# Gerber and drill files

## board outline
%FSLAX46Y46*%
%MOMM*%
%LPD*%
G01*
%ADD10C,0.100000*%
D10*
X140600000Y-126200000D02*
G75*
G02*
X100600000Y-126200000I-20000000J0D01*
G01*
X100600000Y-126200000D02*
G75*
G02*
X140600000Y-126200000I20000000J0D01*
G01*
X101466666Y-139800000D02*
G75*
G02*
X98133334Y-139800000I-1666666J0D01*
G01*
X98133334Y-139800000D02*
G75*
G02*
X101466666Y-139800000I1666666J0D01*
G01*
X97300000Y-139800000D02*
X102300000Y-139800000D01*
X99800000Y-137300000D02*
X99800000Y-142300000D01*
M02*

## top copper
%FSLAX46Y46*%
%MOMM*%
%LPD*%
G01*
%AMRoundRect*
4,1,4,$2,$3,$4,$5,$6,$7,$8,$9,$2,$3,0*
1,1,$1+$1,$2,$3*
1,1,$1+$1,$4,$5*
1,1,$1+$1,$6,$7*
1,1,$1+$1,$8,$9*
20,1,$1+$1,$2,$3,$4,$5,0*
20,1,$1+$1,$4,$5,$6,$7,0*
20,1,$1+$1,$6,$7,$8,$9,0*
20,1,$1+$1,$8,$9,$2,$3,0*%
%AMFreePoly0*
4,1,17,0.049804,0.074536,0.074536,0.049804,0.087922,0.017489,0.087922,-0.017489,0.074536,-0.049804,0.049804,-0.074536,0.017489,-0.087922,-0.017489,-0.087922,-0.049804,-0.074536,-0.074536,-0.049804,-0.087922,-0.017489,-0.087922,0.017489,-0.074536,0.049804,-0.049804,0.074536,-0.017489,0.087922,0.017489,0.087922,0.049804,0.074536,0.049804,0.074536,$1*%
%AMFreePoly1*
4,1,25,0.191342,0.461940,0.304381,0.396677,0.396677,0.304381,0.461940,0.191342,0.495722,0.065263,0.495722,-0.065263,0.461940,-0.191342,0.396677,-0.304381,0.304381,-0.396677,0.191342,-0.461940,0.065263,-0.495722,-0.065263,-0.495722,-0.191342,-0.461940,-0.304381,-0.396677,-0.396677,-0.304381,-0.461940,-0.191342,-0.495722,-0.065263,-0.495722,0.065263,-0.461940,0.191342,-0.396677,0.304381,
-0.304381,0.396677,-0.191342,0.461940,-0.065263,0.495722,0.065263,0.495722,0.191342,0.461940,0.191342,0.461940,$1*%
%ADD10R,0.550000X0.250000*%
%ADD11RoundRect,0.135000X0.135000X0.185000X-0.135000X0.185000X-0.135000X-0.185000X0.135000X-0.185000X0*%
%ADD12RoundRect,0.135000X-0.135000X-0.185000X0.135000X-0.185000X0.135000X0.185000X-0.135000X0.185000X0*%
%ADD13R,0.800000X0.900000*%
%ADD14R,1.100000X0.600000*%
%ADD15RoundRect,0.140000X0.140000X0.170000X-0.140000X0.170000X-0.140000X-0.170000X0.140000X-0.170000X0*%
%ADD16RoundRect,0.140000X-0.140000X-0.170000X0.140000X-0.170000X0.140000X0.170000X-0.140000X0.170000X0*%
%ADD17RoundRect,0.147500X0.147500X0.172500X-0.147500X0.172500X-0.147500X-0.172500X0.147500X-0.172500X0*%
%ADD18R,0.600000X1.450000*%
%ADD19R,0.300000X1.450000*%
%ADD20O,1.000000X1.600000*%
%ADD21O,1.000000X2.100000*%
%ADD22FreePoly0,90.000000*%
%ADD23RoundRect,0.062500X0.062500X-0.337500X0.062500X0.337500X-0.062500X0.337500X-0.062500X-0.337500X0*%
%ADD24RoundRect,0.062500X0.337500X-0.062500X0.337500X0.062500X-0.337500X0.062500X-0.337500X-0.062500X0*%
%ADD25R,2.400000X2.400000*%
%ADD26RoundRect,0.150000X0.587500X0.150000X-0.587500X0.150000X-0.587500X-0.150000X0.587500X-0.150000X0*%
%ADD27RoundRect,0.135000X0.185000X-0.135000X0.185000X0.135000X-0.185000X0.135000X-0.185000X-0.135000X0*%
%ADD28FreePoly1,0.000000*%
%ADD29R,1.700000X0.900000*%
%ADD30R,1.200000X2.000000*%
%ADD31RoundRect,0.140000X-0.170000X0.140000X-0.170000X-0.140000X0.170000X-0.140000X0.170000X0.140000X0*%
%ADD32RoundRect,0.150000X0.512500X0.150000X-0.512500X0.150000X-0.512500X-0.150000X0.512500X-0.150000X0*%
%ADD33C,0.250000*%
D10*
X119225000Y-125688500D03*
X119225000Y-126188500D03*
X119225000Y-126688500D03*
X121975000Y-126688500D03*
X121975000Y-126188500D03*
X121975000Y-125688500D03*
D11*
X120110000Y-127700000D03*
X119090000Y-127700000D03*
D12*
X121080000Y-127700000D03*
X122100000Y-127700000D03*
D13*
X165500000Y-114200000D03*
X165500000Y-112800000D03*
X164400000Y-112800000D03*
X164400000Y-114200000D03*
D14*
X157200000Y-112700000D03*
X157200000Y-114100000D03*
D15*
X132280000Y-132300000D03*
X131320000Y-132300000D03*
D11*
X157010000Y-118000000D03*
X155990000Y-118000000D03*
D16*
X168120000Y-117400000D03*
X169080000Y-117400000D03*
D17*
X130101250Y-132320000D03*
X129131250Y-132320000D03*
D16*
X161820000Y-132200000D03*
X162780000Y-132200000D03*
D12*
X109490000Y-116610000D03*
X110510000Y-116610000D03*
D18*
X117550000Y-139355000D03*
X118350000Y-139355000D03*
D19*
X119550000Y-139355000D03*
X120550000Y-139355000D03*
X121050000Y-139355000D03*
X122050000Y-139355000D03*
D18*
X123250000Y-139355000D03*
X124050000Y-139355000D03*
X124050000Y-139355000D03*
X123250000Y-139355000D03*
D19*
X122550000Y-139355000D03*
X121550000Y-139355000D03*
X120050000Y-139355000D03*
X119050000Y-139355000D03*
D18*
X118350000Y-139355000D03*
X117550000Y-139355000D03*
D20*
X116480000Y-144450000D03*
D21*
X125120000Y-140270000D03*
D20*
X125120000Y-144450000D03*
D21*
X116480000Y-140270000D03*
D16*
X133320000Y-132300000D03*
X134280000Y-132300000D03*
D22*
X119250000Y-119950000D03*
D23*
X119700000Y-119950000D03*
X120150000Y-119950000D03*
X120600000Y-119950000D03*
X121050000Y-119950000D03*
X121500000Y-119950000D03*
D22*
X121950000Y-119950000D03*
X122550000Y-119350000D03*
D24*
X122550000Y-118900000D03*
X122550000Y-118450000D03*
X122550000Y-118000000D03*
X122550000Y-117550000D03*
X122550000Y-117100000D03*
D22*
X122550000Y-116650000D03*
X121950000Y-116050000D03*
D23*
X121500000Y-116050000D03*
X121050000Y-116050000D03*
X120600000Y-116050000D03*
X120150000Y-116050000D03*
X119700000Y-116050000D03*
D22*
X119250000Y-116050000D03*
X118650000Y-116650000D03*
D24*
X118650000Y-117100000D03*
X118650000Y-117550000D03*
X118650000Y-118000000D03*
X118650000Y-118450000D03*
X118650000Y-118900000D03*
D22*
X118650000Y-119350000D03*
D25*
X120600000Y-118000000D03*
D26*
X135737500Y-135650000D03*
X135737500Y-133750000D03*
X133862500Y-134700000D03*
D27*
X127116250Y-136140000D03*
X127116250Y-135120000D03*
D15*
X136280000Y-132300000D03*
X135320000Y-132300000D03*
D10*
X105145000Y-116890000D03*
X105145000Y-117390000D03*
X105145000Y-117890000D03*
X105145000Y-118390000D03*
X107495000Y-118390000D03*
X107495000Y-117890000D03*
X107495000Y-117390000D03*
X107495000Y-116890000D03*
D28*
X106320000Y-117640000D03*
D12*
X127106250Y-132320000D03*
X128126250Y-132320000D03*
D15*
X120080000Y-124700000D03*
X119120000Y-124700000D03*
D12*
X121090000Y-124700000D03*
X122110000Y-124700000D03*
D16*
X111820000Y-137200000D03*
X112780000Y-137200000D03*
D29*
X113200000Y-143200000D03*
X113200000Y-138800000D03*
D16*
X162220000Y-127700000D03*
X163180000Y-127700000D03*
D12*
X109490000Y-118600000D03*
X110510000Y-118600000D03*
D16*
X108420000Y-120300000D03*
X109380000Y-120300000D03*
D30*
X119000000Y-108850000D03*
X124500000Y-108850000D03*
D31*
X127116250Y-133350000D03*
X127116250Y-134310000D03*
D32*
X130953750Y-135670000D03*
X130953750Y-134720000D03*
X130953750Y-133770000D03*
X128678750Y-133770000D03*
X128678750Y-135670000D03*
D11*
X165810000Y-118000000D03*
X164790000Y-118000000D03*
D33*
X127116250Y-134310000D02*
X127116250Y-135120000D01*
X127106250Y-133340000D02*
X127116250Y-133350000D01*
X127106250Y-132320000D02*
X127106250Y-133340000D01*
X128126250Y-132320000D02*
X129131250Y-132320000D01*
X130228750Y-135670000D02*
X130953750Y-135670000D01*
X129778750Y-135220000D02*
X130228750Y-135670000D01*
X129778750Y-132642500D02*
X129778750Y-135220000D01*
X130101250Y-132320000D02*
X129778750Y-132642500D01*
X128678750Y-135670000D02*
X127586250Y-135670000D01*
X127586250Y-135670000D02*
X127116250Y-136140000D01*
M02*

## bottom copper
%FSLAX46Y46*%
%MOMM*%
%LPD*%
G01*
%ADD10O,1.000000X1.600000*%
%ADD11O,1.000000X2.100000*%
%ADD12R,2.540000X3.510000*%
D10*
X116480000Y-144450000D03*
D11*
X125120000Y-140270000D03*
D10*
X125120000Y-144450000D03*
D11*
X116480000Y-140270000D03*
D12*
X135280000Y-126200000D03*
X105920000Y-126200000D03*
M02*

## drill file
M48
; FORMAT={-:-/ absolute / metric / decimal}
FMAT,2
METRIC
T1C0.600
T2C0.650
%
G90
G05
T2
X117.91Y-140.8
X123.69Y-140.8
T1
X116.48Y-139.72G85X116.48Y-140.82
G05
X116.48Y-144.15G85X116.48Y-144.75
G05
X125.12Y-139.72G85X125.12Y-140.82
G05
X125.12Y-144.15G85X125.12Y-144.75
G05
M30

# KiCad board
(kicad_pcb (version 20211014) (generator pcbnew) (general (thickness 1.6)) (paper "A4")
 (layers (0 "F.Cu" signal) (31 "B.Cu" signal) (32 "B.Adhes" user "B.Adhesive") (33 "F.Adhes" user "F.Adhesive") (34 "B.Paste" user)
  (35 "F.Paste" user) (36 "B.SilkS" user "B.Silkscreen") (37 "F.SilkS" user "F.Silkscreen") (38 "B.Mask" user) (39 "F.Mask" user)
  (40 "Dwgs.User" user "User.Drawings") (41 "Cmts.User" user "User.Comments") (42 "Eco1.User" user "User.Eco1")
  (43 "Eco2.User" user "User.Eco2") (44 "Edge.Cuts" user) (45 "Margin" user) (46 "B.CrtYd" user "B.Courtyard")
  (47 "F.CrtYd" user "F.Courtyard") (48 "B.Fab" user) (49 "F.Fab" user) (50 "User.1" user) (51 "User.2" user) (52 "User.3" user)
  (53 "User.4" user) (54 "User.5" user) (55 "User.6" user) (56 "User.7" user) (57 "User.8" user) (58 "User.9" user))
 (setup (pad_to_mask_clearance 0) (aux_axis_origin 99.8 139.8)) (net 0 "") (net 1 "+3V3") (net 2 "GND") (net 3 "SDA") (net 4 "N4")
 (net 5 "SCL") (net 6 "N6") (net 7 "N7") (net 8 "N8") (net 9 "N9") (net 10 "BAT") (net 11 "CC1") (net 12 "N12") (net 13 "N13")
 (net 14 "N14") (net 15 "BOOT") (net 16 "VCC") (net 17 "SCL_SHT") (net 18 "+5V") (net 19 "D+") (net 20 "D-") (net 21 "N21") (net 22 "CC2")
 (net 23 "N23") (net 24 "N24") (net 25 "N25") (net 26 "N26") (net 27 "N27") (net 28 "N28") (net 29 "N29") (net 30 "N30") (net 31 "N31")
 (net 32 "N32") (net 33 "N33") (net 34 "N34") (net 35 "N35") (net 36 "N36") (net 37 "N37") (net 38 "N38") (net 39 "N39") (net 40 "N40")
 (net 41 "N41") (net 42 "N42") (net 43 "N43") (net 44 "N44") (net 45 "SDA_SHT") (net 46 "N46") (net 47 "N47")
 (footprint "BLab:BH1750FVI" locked (layer "F.Cu") (at 120.6 126.1885)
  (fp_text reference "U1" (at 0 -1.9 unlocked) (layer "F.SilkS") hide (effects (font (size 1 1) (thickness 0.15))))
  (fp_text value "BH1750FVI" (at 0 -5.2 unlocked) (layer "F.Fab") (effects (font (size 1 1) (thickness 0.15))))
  (pad "1" smd rect locked (at -1.375 -0.5) (size 0.55 0.25) (layers "F.Cu" "F.Paste" "F.Mask") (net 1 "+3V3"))
  (pad "2" smd rect locked (at -1.375 0) (size 0.55 0.25) (layers "F.Cu" "F.Paste" "F.Mask") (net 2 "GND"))
  (pad "3" smd rect locked (at -1.375 0.5) (size 0.55 0.25) (layers "F.Cu" "F.Paste" "F.Mask") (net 2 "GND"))
  (pad "4" smd rect locked (at 1.375 0.5) (size 0.55 0.25) (layers "F.Cu" "F.Paste" "F.Mask") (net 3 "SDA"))
  (pad "5" smd rect locked (at 1.375 0) (size 0.55 0.25) (layers "F.Cu" "F.Paste" "F.Mask") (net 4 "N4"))
  (pad "6" smd rect locked (at 1.375 -0.5) (size 0.55 0.25) (layers "F.Cu" "F.Paste" "F.Mask") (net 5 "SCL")))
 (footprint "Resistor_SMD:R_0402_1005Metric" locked (layer "F.Cu") (at 119.6 127.7 180)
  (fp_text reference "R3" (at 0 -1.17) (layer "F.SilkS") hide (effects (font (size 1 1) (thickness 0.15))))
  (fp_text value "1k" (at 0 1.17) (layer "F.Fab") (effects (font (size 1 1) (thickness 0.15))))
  (pad "1" smd roundrect locked (at -0.51 0 180) (size 0.54 0.64) (layers "F.Cu" "F.Paste" "F.Mask") (roundrect_rratio 0.25) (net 1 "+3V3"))
  (pad "2" smd roundrect locked (at 0.51 0 180) (size 0.54 0.64) (layers "F.Cu" "F.Paste" "F.Mask") (roundrect_rratio 0.25) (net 4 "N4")))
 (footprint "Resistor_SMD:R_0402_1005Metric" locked (layer "F.Cu") (at 121.59 127.7)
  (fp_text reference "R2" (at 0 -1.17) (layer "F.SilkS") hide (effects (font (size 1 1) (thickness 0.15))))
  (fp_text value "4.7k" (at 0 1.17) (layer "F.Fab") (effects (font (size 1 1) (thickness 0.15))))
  (pad "1" smd roundrect locked (at -0.51 0) (size 0.54 0.64) (layers "F.Cu" "F.Paste" "F.Mask") (roundrect_rratio 0.25) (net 1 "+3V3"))
  (pad "2" smd roundrect locked (at 0.51 0) (size 0.54 0.64) (layers "F.Cu" "F.Paste" "F.Mask") (roundrect_rratio 0.25) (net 3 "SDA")))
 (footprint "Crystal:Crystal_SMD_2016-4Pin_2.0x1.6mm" (layer "F.Cu") (at 164.95 113.5 90)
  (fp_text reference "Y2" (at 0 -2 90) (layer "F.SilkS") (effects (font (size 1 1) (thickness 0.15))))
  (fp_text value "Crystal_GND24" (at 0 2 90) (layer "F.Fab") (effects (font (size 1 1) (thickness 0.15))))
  (pad "1" smd rect (at -0.7 0.55 90) (size 0.9 0.8) (layers "F.Cu" "F.Paste" "F.Mask") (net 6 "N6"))
  (pad "2" smd rect (at 0.7 0.55 90) (size 0.9 0.8) (layers "F.Cu" "F.Paste" "F.Mask") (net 2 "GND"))
  (pad "3" smd rect (at 0.7 -0.55 90) (size 0.9 0.8) (layers "F.Cu" "F.Paste" "F.Mask") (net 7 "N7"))
  (pad "4" smd rect (at -0.7 -0.55 90) (size 0.9 0.8) (layers "F.Cu" "F.Paste" "F.Mask") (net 2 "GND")))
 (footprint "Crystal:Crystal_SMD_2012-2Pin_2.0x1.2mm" (layer "F.Cu") (at 157.2 113.4 -90)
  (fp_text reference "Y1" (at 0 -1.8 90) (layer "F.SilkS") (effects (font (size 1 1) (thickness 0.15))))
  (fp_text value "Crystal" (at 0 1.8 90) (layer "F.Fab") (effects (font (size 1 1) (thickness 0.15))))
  (pad "1" smd rect (at -0.7 0 270) (size 0.6 1.1) (layers "F.Cu" "F.Paste" "F.Mask") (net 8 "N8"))
  (pad "2" smd rect (at 0.7 0 270) (size 0.6 1.1) (layers "F.Cu" "F.Paste" "F.Mask") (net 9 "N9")))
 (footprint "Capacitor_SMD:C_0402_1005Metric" (layer "F.Cu") (at 131.8 132.3 180)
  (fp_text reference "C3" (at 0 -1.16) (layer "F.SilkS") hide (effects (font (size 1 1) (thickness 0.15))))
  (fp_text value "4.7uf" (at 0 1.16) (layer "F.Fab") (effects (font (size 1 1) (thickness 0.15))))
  (pad "1" smd roundrect (at -0.48 0 180) (size 0.56 0.62) (layers "F.Cu" "F.Paste" "F.Mask") (roundrect_rratio 0.25) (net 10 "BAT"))
  (pad "2" smd roundrect (at 0.48 0 180) (size 0.56 0.62) (layers "F.Cu" "F.Paste" "F.Mask") (roundrect_rratio 0.25) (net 2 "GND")))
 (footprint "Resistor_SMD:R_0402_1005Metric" (layer "F.Cu") (at 156.5 118 180)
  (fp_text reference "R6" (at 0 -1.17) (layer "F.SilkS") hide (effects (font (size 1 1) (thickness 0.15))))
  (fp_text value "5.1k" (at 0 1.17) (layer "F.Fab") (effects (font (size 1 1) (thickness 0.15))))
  (pad "1" smd roundrect (at -0.51 0 180) (size 0.54 0.64) (layers "F.Cu" "F.Paste" "F.Mask") (roundrect_rratio 0.25) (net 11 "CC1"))
  (pad "2" smd roundrect (at 0.51 0 180) (size 0.54 0.64) (layers "F.Cu" "F.Paste" "F.Mask") (roundrect_rratio 0.25) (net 2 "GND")))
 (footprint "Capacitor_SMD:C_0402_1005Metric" (layer "F.Cu") (at 168.6 117.4)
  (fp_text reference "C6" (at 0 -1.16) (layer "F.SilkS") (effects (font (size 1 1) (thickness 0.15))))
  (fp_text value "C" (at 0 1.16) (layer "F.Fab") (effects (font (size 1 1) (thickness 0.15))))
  (pad "1" smd roundrect (at -0.48 0) (size 0.56 0.62) (layers "F.Cu" "F.Paste" "F.Mask") (roundrect_rratio 0.25) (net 2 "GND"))
  (pad "2" smd roundrect (at 0.48 0) (size 0.56 0.62) (layers "F.Cu" "F.Paste" "F.Mask") (roundrect_rratio 0.25) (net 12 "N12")))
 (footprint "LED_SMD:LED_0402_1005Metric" (layer "F.Cu") (at 129.61625 132.32 180)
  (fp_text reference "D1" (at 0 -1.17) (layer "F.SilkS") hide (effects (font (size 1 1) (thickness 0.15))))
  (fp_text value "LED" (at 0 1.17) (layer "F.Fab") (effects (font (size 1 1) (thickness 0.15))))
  (pad "1" smd roundrect (at -0.485 0 180) (size 0.59 0.64) (layers "F.Cu" "F.Paste" "F.Mask") (roundrect_rratio 0.25) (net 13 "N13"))
  (pad "2" smd roundrect (at 0.485 0 180) (size 0.59 0.64) (layers "F.Cu" "F.Paste" "F.Mask") (roundrect_rratio 0.25) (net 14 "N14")))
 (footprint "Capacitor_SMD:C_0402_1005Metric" (layer "F.Cu") (at 162.3 132.2)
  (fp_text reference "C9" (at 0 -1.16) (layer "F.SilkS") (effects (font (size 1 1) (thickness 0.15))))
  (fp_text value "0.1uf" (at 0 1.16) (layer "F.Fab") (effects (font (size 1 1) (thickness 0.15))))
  (pad "1" smd roundrect (at -0.48 0) (size 0.56 0.62) (layers "F.Cu" "F.Paste" "F.Mask") (roundrect_rratio 0.25) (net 2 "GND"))
  (pad "2" smd roundrect (at 0.48 0) (size 0.56 0.62) (layers "F.Cu" "F.Paste" "F.Mask") (roundrect_rratio 0.25) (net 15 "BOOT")))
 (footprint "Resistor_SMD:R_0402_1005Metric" (layer "F.Cu") (at 110 116.61)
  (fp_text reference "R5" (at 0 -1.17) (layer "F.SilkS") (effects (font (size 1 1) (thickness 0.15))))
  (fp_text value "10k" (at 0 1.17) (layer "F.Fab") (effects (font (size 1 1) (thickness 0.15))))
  (pad "1" smd roundrect (at -0.51 0) (size 0.54 0.64) (layers "F.Cu" "F.Paste" "F.Mask") (roundrect_rratio 0.25) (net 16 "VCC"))
  (pad "2" smd roundrect (at 0.51 0) (size 0.54 0.64) (layers "F.Cu" "F.Paste" "F.Mask") (roundrect_rratio 0.25) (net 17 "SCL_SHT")))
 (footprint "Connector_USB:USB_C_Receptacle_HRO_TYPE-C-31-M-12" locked (layer "F.Cu") (at 120.8 143.4)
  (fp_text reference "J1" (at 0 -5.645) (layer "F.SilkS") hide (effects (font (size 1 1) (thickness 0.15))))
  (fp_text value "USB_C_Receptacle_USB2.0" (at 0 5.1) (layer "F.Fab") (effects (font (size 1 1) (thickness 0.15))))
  (pad "" np_thru_hole circle locked (at 2.89 -2.6) (size 0.65 0.65) (drill 0.65) (layers *.Cu *.Mask))
  (pad "" np_thru_hole circle locked (at -2.89 -2.6) (size 0.65 0.65) (drill 0.65) (layers *.Cu *.Mask))
  (pad "A1" smd rect locked (at -3.25 -4.045) (size 0.6 1.45) (layers "F.Cu" "F.Paste" "F.Mask") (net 2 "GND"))
  (pad "A4" smd rect locked (at -2.45 -4.045) (size 0.6 1.45) (layers "F.Cu" "F.Paste" "F.Mask") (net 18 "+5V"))
  (pad "A5" smd rect locked (at -1.25 -4.045) (size 0.3 1.45) (layers "F.Cu" "F.Paste" "F.Mask") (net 11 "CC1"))
  (pad "A6" smd rect locked (at -0.25 -4.045) (size 0.3 1.45) (layers "F.Cu" "F.Paste" "F.Mask") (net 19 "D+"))
  (pad "A7" smd rect locked (at 0.25 -4.045) (size 0.3 1.45) (layers "F.Cu" "F.Paste" "F.Mask") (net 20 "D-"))
  (pad "A8" smd rect locked (at 1.25 -4.045) (size 0.3 1.45) (layers "F.Cu" "F.Paste" "F.Mask") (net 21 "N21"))
  (pad "A9" smd rect locked (at 2.45 -4.045) (size 0.6 1.45) (layers "F.Cu" "F.Paste" "F.Mask") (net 18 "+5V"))
  (pad "A12" smd rect locked (at 3.25 -4.045) (size 0.6 1.45) (layers "F.Cu" "F.Paste" "F.Mask") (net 2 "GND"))
  (pad "B1" smd rect locked (at 3.25 -4.045) (size 0.6 1.45) (layers "F.Cu" "F.Paste" "F.Mask") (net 2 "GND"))
  (pad "B4" smd rect locked (at 2.45 -4.045) (size 0.6 1.45) (layers "F.Cu" "F.Paste" "F.Mask") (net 18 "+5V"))
  (pad "B5" smd rect locked (at 1.75 -4.045) (size 0.3 1.45) (layers "F.Cu" "F.Paste" "F.Mask") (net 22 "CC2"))
  (pad "B6" smd rect locked (at 0.75 -4.045) (size 0.3 1.45) (layers "F.Cu" "F.Paste" "F.Mask") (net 19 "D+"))
  (pad "B7" smd rect locked (at -0.75 -4.045) (size 0.3 1.45) (layers "F.Cu" "F.Paste" "F.Mask") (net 20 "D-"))
  (pad "B8" smd rect locked (at -1.75 -4.045) (size 0.3 1.45) (layers "F.Cu" "F.Paste" "F.Mask") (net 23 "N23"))
  (pad "B9" smd rect locked (at -2.45 -4.045) (size 0.6 1.45) (layers "F.Cu" "F.Paste" "F.Mask") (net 18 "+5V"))
  (pad "B12" smd rect locked (at -3.25 -4.045) (size 0.6 1.45) (layers "F.Cu" "F.Paste" "F.Mask") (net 2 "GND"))
  (pad "S1" thru_hole oval locked (at -4.32 1.05) (size 1 1.6) (drill oval 0.6 1.2) (layers *.Cu *.Mask) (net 2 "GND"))
  (pad "S1" thru_hole oval locked (at 4.32 -3.13) (size 1 2.1) (drill oval 0.6 1.7) (layers *.Cu *.Mask) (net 2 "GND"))
  (pad "S1" thru_hole oval locked (at 4.32 1.05) (size 1 1.6) (drill oval 0.6 1.2) (layers *.Cu *.Mask) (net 2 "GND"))
  (pad "S1" thru_hole oval locked (at -4.32 -3.13) (size 1 2.1) (drill oval 0.6 1.7) (layers *.Cu *.Mask) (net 2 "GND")))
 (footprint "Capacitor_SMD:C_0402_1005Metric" (layer "F.Cu") (at 133.8 132.3)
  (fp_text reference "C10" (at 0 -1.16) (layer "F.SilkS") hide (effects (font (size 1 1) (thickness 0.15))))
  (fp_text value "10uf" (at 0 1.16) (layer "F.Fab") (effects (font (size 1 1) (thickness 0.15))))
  (pad "1" smd roundrect (at -0.48 0) (size 0.56 0.62) (layers "F.Cu" "F.Paste" "F.Mask") (roundrect_rratio 0.25) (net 10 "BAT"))
  (pad "2" smd roundrect (at 0.48 0) (size 0.56 0.62) (layers "F.Cu" "F.Paste" "F.Mask") (roundrect_rratio 0.25) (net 2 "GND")))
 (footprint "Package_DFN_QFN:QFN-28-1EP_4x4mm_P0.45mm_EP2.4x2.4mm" (layer "F.Cu") (at 120.6 118 90)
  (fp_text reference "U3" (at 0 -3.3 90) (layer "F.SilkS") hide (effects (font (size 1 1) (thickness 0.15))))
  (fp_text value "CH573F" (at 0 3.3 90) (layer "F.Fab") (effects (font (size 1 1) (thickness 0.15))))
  (pad "" smd roundrect (at 0.6 -0.6 90) (size 0.97 0.97) (layers "F.Paste") (roundrect_rratio 0.25))
  (pad "" smd roundrect (at -0.6 0.6 90) (size 0.97 0.97) (layers "F.Paste") (roundrect_rratio 0.25))
  (pad "" smd roundrect (at 0.6 0.6 90) (size 0.97 0.97) (layers "F.Paste") (roundrect_rratio 0.25))
  (pad "" smd roundrect (at -0.6 -0.6 90) (size 0.97 0.97) (layers "F.Paste") (roundrect_rratio 0.25))
  (pad "1" smd custom (at -1.95 -1.35 90) (size 0.179289 0.179289) (layers "F.Cu" "F.Paste" "F.Mask") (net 8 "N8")
   (options (clearance outline) (anchor circle)) (primitives))
  (pad "2" smd roundrect (at -1.95 -0.9 90) (size 0.8 0.25) (layers "F.Cu" "F.Paste" "F.Mask") (roundrect_rratio 0.25) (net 9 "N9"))
  (pad "3" smd roundrect (at -1.95 -0.45 90) (size 0.8 0.25) (layers "F.Cu" "F.Paste" "F.Mask") (roundrect_rratio 0.25) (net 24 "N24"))
  (pad "4" smd roundrect (at -1.95 0 90) (size 0.8 0.25) (layers "F.Cu" "F.Paste" "F.Mask") (roundrect_rratio 0.25) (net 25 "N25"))
  (pad "5" smd roundrect (at -1.95 0.45 90) (size 0.8 0.25) (layers "F.Cu" "F.Paste" "F.Mask") (roundrect_rratio 0.25) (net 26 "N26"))
  (pad "6" smd roundrect (at -1.95 0.9 90) (size 0.8 0.25) (layers "F.Cu" "F.Paste" "F.Mask") (roundrect_rratio 0.25) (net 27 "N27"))
  (pad "7" smd custom (at -1.95 1.35 90) (size 0.179289 0.179289) (layers "F.Cu" "F.Paste" "F.Mask") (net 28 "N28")
   (options (clearance outline) (anchor circle)) (primitives))
  (pad "8" smd custom (at -1.35 1.95 90) (size 0.179289 0.179289) (layers "F.Cu" "F.Paste" "F.Mask") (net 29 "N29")
   (options (clearance outline) (anchor circle)) (primitives))
  (pad "9" smd roundrect (at -0.9 1.95 90) (size 0.25 0.8) (layers "F.Cu" "F.Paste" "F.Mask") (roundrect_rratio 0.25) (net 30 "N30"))
  (pad "10" smd roundrect (at -0.45 1.95 90) (size 0.25 0.8) (layers "F.Cu" "F.Paste" "F.Mask") (roundrect_rratio 0.25) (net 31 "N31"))
  (pad "11" smd roundrect (at 0 1.95 90) (size 0.25 0.8) (layers "F.Cu" "F.Paste" "F.Mask") (roundrect_rratio 0.25) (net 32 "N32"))
  (pad "12" smd roundrect (at 0.45 1.95 90) (size 0.25 0.8) (layers "F.Cu" "F.Paste" "F.Mask") (roundrect_rratio 0.25) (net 19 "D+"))
  (pad "13" smd roundrect (at 0.9 1.95 90) (size 0.25 0.8) (layers "F.Cu" "F.Paste" "F.Mask") (roundrect_rratio 0.25) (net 20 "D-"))
  (pad "14" smd custom (at 1.35 1.95 90) (size 0.179289 0.179289) (layers "F.Cu" "F.Paste" "F.Mask") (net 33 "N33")
   (options (clearance outline) (anchor circle)) (primitives))
  (pad "15" smd custom (at 1.95 1.35 90) (size 0.179289 0.179289) (layers "F.Cu" "F.Paste" "F.Mask") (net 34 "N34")
   (options (clearance outline) (anchor circle)) (primitives))
  (pad "16" smd roundrect (at 1.95 0.9 90) (size 0.8 0.25) (layers "F.Cu" "F.Paste" "F.Mask") (roundrect_rratio 0.25) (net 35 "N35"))
  (pad "17" smd roundrect (at 1.95 0.45 90) (size 0.8 0.25) (layers "F.Cu" "F.Paste" "F.Mask") (roundrect_rratio 0.25) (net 15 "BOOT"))
  (pad "18" smd roundrect (at 1.95 0 90) (size 0.8 0.25) (layers "F.Cu" "F.Paste" "F.Mask") (roundrect_rratio 0.25) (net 6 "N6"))
  (pad "19" smd roundrect (at 1.95 -0.45 90) (size 0.8 0.25) (layers "F.Cu" "F.Paste" "F.Mask") (roundrect_rratio 0.25) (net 7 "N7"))
  (pad "20" smd roundrect (at 1.95 -0.9 90) (size 0.8 0.25) (layers "F.Cu" "F.Paste" "F.Mask") (roundrect_rratio 0.25) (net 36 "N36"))
  (pad "21" smd custom (at 1.95 -1.35 90) (size 0.179289 0.179289) (layers "F.Cu" "F.Paste" "F.Mask") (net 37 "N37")
   (options (clearance outline) (anchor circle)) (primitives))
  (pad "22" smd custom (at 1.35 -1.95 90) (size 0.179289 0.179289) (layers "F.Cu" "F.Paste" "F.Mask") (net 12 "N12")
   (options (clearance outline) (anchor circle)) (primitives))
  (pad "23" smd roundrect (at 0.9 -1.95 90) (size 0.25 0.8) (layers "F.Cu" "F.Paste" "F.Mask") (roundrect_rratio 0.25) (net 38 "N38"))
  (pad "24" smd roundrect (at 0.45 -1.95 90) (size 0.25 0.8) (layers "F.Cu" "F.Paste" "F.Mask") (roundrect_rratio 0.25) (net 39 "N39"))
  (pad "25" smd roundrect (at 0 -1.95 90) (size 0.25 0.8) (layers "F.Cu" "F.Paste" "F.Mask") (roundrect_rratio 0.25) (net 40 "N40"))
  (pad "26" smd roundrect (at -0.45 -1.95 90) (size 0.25 0.8) (layers "F.Cu" "F.Paste" "F.Mask") (roundrect_rratio 0.25) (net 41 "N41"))
  (pad "27" smd roundrect (at -0.9 -1.95 90) (size 0.25 0.8) (layers "F.Cu" "F.Paste" "F.Mask") (roundrect_rratio 0.25) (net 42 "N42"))
  (pad "28" smd custom (at -1.35 -1.95 90) (size 0.179289 0.179289) (layers "F.Cu" "F.Paste" "F.Mask") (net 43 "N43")
   (options (clearance outline) (anchor circle)) (primitives))
  (pad "29" smd rect (at 0 0 90) (size 2.4 2.4) (layers "F.Cu" "F.Mask") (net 2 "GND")))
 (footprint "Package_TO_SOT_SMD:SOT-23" (layer "F.Cu") (at 134.8 134.7 180)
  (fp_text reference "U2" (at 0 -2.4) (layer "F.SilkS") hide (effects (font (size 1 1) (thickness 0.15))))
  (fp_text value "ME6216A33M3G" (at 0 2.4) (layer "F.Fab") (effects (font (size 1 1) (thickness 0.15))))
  (pad "1" smd roundrect (at -0.9375 -0.95 180) (size 1.475 0.6) (layers "F.Cu" "F.Paste" "F.Mask") (roundrect_rratio 0.25) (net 2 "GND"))
  (pad "2" smd roundrect (at -0.9375 0.95 180) (size 1.475 0.6) (layers "F.Cu" "F.Paste" "F.Mask") (roundrect_rratio 0.25) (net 16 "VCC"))
  (pad "3" smd roundrect (at 0.9375 0 180) (size 1.475 0.6) (layers "F.Cu" "F.Paste" "F.Mask") (roundrect_rratio 0.25) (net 10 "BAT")))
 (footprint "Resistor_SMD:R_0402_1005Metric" (layer "F.Cu") (at 127.11625 135.63 90)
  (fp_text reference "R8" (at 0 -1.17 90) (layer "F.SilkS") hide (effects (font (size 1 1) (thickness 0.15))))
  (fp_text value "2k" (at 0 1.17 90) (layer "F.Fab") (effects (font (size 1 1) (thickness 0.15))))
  (pad "1" smd roundrect (at -0.51 0 90) (size 0.54 0.64) (layers "F.Cu" "F.Paste" "F.Mask") (roundrect_rratio 0.25) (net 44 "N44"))
  (pad "2" smd roundrect (at 0.51 0 90) (size 0.54 0.64) (layers "F.Cu" "F.Paste" "F.Mask") (roundrect_rratio 0.25) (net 2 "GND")))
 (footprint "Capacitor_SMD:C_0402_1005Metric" (layer "F.Cu") (at 135.8 132.3 180)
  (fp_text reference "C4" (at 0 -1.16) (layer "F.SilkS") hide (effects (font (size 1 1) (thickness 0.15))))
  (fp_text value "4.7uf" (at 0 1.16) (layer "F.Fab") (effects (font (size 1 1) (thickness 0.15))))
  (pad "1" smd roundrect (at -0.48 0 180) (size 0.56 0.62) (layers "F.Cu" "F.Paste" "F.Mask") (roundrect_rratio 0.25) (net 16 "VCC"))
  (pad "2" smd roundrect (at 0.48 0 180) (size 0.56 0.62) (layers "F.Cu" "F.Paste" "F.Mask") (roundrect_rratio 0.25) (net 2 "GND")))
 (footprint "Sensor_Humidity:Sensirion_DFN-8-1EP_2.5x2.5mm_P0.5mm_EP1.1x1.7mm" (layer "F.Cu") (at 106.32 117.64)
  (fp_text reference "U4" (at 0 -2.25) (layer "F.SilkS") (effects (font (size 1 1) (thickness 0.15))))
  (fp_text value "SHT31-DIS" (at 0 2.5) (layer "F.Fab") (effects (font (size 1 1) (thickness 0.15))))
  (pad "" smd custom (at 0 0) (size 0.9 0.9) (layers "F.Paste") (zone_connect 0) (options (clearance outline) (anchor rect)) (primitives))
  (pad "1" smd rect (at -1.175 -0.75) (size 0.55 0.25) (layers "F.Cu" "F.Paste" "F.Mask") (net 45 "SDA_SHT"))
  (pad "2" smd rect (at -1.175 -0.25) (size 0.55 0.25) (layers "F.Cu" "F.Paste" "F.Mask") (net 2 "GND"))
  (pad "3" smd rect (at -1.175 0.25) (size 0.55 0.25) (layers "F.Cu" "F.Paste" "F.Mask") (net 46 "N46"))
  (pad "4" smd rect (at -1.175 0.75 180) (size 0.55 0.25) (layers "F.Cu" "F.Paste" "F.Mask") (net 17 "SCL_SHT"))
  (pad "5" smd rect (at 1.175 0.75) (size 0.55 0.25) (layers "F.Cu" "F.Paste" "F.Mask") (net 16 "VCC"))
  (pad "6" smd rect (at 1.175 0.25) (size 0.55 0.25) (layers "F.Cu" "F.Paste" "F.Mask") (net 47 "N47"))
  (pad "7" smd rect (at 1.175 -0.25) (size 0.55 0.25) (layers "F.Cu" "F.Paste" "F.Mask") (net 2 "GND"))
  (pad "8" smd rect (at 1.175 -0.75) (size 0.55 0.25) (layers "F.Cu" "F.Paste" "F.Mask") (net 2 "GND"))
  (pad "9" smd custom (at 0 0) (size 1 1) (layers "F.Cu" "F.Mask") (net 2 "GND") (zone_connect 0)
   (options (clearance outline) (anchor circle)) (primitives)))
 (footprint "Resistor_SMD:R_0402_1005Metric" (layer "F.Cu") (at 127.61625 132.32)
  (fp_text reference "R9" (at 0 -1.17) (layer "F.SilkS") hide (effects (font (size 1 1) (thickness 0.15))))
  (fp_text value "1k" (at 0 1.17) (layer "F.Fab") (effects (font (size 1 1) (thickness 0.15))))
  (pad "1" smd roundrect (at -0.51 0) (size 0.54 0.64) (layers "F.Cu" "F.Paste" "F.Mask") (roundrect_rratio 0.25) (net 18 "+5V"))
  (pad "2" smd roundrect (at 0.51 0) (size 0.54 0.64) (layers "F.Cu" "F.Paste" "F.Mask") (roundrect_rratio 0.25) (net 14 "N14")))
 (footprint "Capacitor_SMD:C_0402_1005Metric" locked (layer "F.Cu") (at 119.6 124.7 180)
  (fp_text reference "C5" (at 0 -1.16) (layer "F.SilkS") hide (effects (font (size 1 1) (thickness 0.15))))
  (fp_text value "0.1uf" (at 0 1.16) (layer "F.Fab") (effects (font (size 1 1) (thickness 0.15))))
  (pad "1" smd roundrect locked (at -0.48 0 180) (size 0.56 0.62) (layers "F.Cu" "F.Paste" "F.Mask") (roundrect_rratio 0.25) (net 4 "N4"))
  (pad "2" smd roundrect locked (at 0.48 0 180) (size 0.56 0.62) (layers "F.Cu" "F.Paste" "F.Mask") (roundrect_rratio 0.25) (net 2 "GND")))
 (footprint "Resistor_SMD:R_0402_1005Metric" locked (layer "F.Cu") (at 121.6 124.7)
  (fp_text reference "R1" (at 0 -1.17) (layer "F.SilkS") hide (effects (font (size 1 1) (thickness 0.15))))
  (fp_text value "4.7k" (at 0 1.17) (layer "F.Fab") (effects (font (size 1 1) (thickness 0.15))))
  (pad "1" smd roundrect locked (at -0.51 0) (size 0.54 0.64) (layers "F.Cu" "F.Paste" "F.Mask") (roundrect_rratio 0.25) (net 1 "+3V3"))
  (pad "2" smd roundrect locked (at 0.51 0) (size 0.54 0.64) (layers "F.Cu" "F.Paste" "F.Mask") (roundrect_rratio 0.25) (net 5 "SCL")))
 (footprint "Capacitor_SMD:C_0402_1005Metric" (layer "F.Cu") (at 112.3 137.2)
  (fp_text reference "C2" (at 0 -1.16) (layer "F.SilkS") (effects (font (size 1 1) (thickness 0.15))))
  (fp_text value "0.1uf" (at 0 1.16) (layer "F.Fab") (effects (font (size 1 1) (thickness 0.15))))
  (pad "1" smd roundrect (at -0.48 0) (size 0.56 0.62) (layers "F.Cu" "F.Paste" "F.Mask") (roundrect_rratio 0.25) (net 2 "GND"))
  (pad "2" smd roundrect (at 0.48 0) (size 0.56 0.62) (layers "F.Cu" "F.Paste" "F.Mask") (roundrect_rratio 0.25) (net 26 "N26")))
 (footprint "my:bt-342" (layer "F.Cu") (at 113.2 141 90)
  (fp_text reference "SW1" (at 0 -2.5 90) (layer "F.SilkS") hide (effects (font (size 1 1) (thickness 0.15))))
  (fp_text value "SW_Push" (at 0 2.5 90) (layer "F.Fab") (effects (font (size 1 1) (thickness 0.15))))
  (pad "1" smd rect locked (at -2.2 0 90) (size 0.9 1.7) (layers "F.Cu" "F.Paste" "F.Mask") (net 15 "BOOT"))
  (pad "2" smd rect locked (at 2.2 0 90) (size 0.9 1.7) (layers "F.Cu" "F.Paste" "F.Mask") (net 2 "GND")))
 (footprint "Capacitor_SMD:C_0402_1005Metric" (layer "F.Cu") (at 162.7 127.7)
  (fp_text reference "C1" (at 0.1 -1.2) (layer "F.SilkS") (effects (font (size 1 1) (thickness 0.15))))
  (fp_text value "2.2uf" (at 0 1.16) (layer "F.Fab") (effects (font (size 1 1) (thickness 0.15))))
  (pad "1" smd roundrect (at -0.48 0) (size 0.56 0.62) (layers "F.Cu" "F.Paste" "F.Mask") (roundrect_rratio 0.25) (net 2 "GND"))
  (pad "2" smd roundrect (at 0.48 0) (size 0.56 0.62) (layers "F.Cu" "F.Paste" "F.Mask") (roundrect_rratio 0.25) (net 24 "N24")))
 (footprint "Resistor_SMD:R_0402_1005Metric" (layer "F.Cu") (at 110 118.6)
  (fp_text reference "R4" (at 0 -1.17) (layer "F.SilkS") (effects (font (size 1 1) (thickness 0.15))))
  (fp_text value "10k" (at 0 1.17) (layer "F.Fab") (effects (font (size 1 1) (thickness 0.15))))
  (pad "1" smd roundrect (at -0.51 0) (size 0.54 0.64) (layers "F.Cu" "F.Paste" "F.Mask") (roundrect_rratio 0.25) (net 16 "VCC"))
  (pad "2" smd roundrect (at 0.51 0) (size 0.54 0.64) (layers "F.Cu" "F.Paste" "F.Mask") (roundrect_rratio 0.25) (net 45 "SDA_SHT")))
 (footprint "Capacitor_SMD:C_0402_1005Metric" (layer "F.Cu") (at 108.9 120.3)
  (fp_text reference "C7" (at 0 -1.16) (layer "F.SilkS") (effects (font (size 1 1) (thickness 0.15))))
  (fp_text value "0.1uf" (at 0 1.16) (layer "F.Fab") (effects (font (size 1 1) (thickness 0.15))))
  (pad "1" smd roundrect (at -0.48 0) (size 0.56 0.62) (layers "F.Cu" "F.Paste" "F.Mask") (roundrect_rratio 0.25) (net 16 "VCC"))
  (pad "2" smd roundrect (at 0.48 0) (size 0.56 0.62) (layers "F.Cu" "F.Paste" "F.Mask") (roundrect_rratio 0.25) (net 2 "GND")))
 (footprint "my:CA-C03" (layer "F.Cu") (at 119 108.85)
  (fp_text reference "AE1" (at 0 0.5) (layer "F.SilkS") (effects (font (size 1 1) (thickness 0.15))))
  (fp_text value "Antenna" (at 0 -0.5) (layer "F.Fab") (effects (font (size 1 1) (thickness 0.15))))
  (pad "1" smd rect locked (at 0 0) (size 1.2 2) (layers "F.Cu" "F.Paste" "F.Mask") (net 37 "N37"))
  (pad "2" smd rect locked (at 5.5 0) (size 1.2 2) (layers "F.Cu" "F.Paste" "F.Mask")))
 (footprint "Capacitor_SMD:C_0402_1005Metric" (layer "F.Cu") (at 127.11625 133.83 -90)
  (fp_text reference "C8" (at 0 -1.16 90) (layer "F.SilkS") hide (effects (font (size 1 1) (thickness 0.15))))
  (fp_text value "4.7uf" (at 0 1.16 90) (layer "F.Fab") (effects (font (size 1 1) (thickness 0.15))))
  (pad "1" smd roundrect (at -0.48 0 270) (size 0.56 0.62) (layers "F.Cu" "F.Paste" "F.Mask") (roundrect_rratio 0.25) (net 18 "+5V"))
  (pad "2" smd roundrect (at 0.48 0 270) (size 0.56 0.62) (layers "F.Cu" "F.Paste" "F.Mask") (roundrect_rratio 0.25) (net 2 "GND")))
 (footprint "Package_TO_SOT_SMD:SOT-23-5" (layer "F.Cu") (at 129.81625 134.72 180)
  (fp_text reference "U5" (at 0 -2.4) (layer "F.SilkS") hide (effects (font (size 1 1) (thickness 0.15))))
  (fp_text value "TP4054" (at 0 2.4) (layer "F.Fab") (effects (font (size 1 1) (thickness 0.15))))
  (pad "1" smd roundrect (at -1.1375 -0.95 180) (size 1.325 0.6) (layers "F.Cu" "F.Paste" "F.Mask") (roundrect_rratio 0.25) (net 13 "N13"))
  (pad "2" smd roundrect (at -1.1375 0 180) (size 1.325 0.6) (layers "F.Cu" "F.Paste" "F.Mask") (roundrect_rratio 0.25) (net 2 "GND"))
  (pad "3" smd roundrect (at -1.1375 0.95 180) (size 1.325 0.6) (layers "F.Cu" "F.Paste" "F.Mask") (roundrect_rratio 0.25) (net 10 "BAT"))
  (pad "4" smd roundrect (at 1.1375 0.95 180) (size 1.325 0.6) (layers "F.Cu" "F.Paste" "F.Mask") (roundrect_rratio 0.25) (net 18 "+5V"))
  (pad "5" smd roundrect (at 1.1375 -0.95 180) (size 1.325 0.6) (layers "F.Cu" "F.Paste" "F.Mask") (roundrect_rratio 0.25) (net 44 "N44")))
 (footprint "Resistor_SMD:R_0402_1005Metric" (layer "F.Cu") (at 165.3 118 180)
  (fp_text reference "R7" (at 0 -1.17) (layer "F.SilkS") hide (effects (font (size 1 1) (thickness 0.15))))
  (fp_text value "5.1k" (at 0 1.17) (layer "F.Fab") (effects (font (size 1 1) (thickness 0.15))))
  (pad "1" smd roundrect (at -0.51 0 180) (size 0.54 0.64) (layers "F.Cu" "F.Paste" "F.Mask") (roundrect_rratio 0.25) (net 22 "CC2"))
  (pad "2" smd roundrect (at 0.51 0 180) (size 0.54 0.64) (layers "F.Cu" "F.Paste" "F.Mask") (roundrect_rratio 0.25) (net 2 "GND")))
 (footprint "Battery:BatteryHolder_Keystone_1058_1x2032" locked (layer "B.Cu") (at 120.6 126.2 180)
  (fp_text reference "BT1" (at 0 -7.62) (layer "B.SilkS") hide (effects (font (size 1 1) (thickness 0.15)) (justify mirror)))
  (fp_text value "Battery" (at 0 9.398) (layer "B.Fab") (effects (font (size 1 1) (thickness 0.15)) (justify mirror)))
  (pad "1" smd rect locked (at -14.68 0 180) (size 2.54 3.51) (layers "B.Cu" "B.Paste" "B.Mask") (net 10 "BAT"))
  (pad "2" smd rect locked (at 14.68 0 180) (size 2.54 3.51) (layers "B.Cu" "B.Paste" "B.Mask") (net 2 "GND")))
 (gr_circle (center 120.6 126.2) (end 140.6 126.2) (layer "Edge.Cuts") (width 0.1) (fill none))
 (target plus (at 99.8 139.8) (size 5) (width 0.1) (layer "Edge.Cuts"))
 (segment (start 127.11625 134.31) (end 127.11625 135.12) (width 0.25) (layer "F.Cu") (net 2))
 (segment (start 127.10625 133.34) (end 127.11625 133.35) (width 0.25) (layer "F.Cu") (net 18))
 (segment (start 127.10625 132.32) (end 127.10625 133.34) (width 0.25) (layer "F.Cu") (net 18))
 (segment (start 128.12625 132.32) (end 129.13125 132.32) (width 0.25) (layer "F.Cu") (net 14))
 (segment (start 130.22875 135.67) (end 130.95375 135.67) (width 0.25) (layer "F.Cu") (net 13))
 (segment (start 129.77875 135.22) (end 130.22875 135.67) (width 0.25) (layer "F.Cu") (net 13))
 (segment (start 129.77875 132.6425) (end 129.77875 135.22) (width 0.25) (layer "F.Cu") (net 13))
 (segment (start 130.10125 132.32) (end 129.77875 132.6425) (width 0.25) (layer "F.Cu") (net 13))
 (segment (start 128.67875 135.67) (end 127.58625 135.67) (width 0.25) (layer "F.Cu") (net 44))
 (segment (start 127.58625 135.67) (end 127.11625 136.14) (width 0.25) (layer "F.Cu") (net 44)))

